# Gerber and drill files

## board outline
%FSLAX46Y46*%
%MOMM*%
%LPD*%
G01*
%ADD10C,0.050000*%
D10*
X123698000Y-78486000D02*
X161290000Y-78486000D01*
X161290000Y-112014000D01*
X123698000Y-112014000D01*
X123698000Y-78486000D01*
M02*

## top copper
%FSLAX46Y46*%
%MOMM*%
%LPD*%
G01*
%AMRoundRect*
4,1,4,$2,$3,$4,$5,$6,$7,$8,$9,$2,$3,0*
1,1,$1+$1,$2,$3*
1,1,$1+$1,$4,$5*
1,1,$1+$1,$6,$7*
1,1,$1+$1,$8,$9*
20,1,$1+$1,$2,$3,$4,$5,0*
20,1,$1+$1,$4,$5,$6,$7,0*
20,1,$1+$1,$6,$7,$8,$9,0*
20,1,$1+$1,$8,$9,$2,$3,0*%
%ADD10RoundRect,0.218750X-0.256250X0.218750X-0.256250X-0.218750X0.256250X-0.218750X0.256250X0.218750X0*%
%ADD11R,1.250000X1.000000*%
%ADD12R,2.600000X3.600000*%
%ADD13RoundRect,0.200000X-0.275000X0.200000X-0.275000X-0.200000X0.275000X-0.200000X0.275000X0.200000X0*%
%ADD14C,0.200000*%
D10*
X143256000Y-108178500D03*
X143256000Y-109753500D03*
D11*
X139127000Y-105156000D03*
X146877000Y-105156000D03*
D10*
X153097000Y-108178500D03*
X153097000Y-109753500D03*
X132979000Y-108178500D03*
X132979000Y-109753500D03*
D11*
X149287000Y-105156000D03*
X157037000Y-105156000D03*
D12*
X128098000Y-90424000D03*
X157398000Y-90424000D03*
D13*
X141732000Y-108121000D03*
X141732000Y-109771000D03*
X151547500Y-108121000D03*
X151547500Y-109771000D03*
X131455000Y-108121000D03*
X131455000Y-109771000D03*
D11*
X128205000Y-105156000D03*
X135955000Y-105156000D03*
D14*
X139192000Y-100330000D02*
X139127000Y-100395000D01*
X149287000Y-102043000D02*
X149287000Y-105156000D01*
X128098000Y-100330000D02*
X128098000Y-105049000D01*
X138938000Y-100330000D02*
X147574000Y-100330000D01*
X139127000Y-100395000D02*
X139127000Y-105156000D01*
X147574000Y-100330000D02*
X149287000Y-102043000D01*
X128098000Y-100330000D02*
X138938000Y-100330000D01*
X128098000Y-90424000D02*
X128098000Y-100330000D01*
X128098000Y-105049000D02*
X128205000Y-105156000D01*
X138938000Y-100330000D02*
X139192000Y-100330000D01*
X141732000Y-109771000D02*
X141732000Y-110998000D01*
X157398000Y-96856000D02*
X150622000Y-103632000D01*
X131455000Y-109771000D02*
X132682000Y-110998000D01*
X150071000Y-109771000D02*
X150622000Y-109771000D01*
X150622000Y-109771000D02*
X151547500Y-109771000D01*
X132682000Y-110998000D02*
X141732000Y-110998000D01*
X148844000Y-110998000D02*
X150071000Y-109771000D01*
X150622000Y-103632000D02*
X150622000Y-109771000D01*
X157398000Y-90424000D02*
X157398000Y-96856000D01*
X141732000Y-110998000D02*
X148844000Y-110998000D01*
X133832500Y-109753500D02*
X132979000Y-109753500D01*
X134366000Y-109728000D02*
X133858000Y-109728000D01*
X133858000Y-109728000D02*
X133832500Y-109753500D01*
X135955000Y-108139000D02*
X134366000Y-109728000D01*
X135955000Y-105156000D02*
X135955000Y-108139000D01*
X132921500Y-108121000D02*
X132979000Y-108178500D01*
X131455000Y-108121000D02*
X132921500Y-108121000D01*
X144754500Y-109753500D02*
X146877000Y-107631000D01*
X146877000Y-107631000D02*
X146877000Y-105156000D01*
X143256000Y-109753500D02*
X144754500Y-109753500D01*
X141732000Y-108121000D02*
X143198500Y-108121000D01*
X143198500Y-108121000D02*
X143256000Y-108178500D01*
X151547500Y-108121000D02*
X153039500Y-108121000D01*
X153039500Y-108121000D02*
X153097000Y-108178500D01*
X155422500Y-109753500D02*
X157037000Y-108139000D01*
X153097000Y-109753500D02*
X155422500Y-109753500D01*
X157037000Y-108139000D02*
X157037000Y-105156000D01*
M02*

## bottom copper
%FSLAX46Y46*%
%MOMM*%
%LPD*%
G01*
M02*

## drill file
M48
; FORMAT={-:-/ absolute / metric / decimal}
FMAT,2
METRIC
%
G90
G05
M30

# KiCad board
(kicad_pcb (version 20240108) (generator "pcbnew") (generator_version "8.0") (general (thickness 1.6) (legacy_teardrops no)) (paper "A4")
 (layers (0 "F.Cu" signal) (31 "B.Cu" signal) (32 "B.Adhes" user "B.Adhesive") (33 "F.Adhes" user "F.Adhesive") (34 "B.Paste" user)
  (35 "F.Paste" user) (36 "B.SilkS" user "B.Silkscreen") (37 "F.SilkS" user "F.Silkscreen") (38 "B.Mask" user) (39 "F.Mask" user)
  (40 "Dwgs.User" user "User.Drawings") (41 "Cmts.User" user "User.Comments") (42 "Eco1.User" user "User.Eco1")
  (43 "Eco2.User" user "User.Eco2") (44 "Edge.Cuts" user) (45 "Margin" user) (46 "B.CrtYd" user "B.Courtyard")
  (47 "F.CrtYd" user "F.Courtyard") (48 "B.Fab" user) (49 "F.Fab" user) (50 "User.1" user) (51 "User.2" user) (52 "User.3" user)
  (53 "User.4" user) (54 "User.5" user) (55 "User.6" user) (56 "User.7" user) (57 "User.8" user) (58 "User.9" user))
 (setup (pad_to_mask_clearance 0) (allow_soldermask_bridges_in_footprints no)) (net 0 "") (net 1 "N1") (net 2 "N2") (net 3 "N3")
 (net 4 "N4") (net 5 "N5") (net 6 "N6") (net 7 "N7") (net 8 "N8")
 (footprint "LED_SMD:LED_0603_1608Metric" (layer "F.Cu") (at 143.256 108.966 -90)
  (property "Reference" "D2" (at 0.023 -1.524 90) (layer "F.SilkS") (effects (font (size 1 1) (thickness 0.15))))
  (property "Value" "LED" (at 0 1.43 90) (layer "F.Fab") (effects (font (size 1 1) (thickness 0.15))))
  (pad "1" smd roundrect (at -0.7875 0 270) (size 0.875 0.95) (layers "F.Cu" "F.Paste" "F.Mask") (roundrect_rratio 0.25) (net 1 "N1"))
  (pad "2" smd roundrect (at 0.7875 0 270) (size 0.875 0.95) (layers "F.Cu" "F.Paste" "F.Mask") (roundrect_rratio 0.25) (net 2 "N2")))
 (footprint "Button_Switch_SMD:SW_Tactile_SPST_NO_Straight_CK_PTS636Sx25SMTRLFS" (layer "F.Cu") (at 143.002 105.156)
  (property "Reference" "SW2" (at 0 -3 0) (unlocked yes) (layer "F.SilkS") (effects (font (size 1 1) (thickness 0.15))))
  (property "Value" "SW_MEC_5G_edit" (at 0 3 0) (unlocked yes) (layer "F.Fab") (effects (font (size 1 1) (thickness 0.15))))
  (pad "1" smd rect (at -3.875 0) (size 1.25 1) (layers "F.Cu" "F.Paste" "F.Mask") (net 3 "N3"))
  (pad "2" smd rect (at 3.875 0) (size 1.25 1) (layers "F.Cu" "F.Paste" "F.Mask") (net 2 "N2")))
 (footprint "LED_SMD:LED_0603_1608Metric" (layer "F.Cu") (at 153.097 108.966 -90)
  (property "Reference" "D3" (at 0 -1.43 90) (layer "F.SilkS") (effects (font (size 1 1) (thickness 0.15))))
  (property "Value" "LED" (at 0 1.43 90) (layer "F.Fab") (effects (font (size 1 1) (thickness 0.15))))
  (pad "1" smd roundrect (at -0.7875 0 270) (size 0.875 0.95) (layers "F.Cu" "F.Paste" "F.Mask") (roundrect_rratio 0.25) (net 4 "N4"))
  (pad "2" smd roundrect (at 0.7875 0 270) (size 0.875 0.95) (layers "F.Cu" "F.Paste" "F.Mask") (roundrect_rratio 0.25) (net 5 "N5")))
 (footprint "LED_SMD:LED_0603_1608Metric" (layer "F.Cu") (at 132.979 108.966 -90)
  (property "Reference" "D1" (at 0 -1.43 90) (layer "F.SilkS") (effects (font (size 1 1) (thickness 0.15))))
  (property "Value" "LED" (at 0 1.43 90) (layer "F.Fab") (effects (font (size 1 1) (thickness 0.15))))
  (pad "1" smd roundrect (at -0.7875 0 270) (size 0.875 0.95) (layers "F.Cu" "F.Paste" "F.Mask") (roundrect_rratio 0.25) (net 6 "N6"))
  (pad "2" smd roundrect (at 0.7875 0 270) (size 0.875 0.95) (layers "F.Cu" "F.Paste" "F.Mask") (roundrect_rratio 0.25) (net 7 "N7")))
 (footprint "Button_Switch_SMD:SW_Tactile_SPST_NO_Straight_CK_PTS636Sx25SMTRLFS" (layer "F.Cu") (at 153.162 105.156)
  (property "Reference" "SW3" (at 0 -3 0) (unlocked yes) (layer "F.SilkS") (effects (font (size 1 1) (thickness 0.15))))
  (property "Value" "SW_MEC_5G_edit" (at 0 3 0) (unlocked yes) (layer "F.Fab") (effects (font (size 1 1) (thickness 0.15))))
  (pad "1" smd rect (at -3.875 0) (size 1.25 1) (layers "F.Cu" "F.Paste" "F.Mask") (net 3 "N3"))
  (pad "2" smd rect (at 3.875 0) (size 1.25 1) (layers "F.Cu" "F.Paste" "F.Mask") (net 5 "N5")))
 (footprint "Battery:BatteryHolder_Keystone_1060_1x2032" (layer "F.Cu") (at 142.748 90.424)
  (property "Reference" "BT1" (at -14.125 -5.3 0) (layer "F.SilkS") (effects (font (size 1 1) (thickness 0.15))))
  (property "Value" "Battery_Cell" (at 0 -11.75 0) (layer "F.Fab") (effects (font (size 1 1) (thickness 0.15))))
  (pad "1" smd rect (at -14.65 0 180) (size 2.6 3.6) (layers "F.Cu" "F.Paste" "F.Mask") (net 3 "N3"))
  (pad "2" smd rect (at 14.65 0 180) (size 2.6 3.6) (layers "F.Cu" "F.Paste" "F.Mask") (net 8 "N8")))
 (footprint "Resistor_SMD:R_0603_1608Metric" (layer "F.Cu") (at 141.732 108.946 -90)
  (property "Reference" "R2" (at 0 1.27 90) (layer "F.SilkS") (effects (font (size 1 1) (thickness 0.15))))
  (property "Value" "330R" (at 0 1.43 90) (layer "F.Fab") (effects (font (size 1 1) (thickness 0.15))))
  (pad "1" smd roundrect (at -0.825 0 270) (size 0.8 0.95) (layers "F.Cu" "F.Paste" "F.Mask") (roundrect_rratio 0.25) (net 1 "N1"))
  (pad "2" smd roundrect (at 0.825 0 270) (size 0.8 0.95) (layers "F.Cu" "F.Paste" "F.Mask") (roundrect_rratio 0.25) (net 8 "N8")))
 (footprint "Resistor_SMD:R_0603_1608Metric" (layer "F.Cu") (at 151.5475 108.946 -90)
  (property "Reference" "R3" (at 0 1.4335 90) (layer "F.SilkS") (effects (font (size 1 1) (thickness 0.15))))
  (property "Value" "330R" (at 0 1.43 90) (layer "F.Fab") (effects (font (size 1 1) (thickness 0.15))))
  (pad "1" smd roundrect (at -0.825 0 270) (size 0.8 0.95) (layers "F.Cu" "F.Paste" "F.Mask") (roundrect_rratio 0.25) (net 4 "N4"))
  (pad "2" smd roundrect (at 0.825 0 270) (size 0.8 0.95) (layers "F.Cu" "F.Paste" "F.Mask") (roundrect_rratio 0.25) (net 8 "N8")))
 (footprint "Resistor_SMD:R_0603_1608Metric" (layer "F.Cu") (at 131.455 108.946 -90)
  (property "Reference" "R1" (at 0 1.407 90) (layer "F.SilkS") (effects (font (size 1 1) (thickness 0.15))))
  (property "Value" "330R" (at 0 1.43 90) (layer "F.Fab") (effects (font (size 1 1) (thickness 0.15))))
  (pad "1" smd roundrect (at -0.825 0 270) (size 0.8 0.95) (layers "F.Cu" "F.Paste" "F.Mask") (roundrect_rratio 0.25) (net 6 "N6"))
  (pad "2" smd roundrect (at 0.825 0 270) (size 0.8 0.95) (layers "F.Cu" "F.Paste" "F.Mask") (roundrect_rratio 0.25) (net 8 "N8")))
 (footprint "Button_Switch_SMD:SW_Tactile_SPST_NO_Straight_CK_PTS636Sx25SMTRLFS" (layer "F.Cu") (at 132.08 105.156)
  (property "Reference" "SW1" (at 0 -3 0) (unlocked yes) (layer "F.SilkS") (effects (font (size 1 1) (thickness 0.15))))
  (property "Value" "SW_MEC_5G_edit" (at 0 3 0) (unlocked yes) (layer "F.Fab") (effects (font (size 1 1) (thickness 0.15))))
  (pad "1" smd rect (at -3.875 0) (size 1.25 1) (layers "F.Cu" "F.Paste" "F.Mask") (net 3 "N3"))
  (pad "2" smd rect (at 3.875 0) (size 1.25 1) (layers "F.Cu" "F.Paste" "F.Mask") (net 7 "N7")))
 (gr_rect (start 123.698 78.486) (end 161.29 112.014) (stroke (width 0.05) (type default)) (fill none) (layer "Edge.Cuts"))
 (segment (start 139.192 100.33) (end 139.127 100.395) (width 0.2) (layer "F.Cu") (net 3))
 (segment (start 149.287 102.043) (end 149.287 105.156) (width 0.2) (layer "F.Cu") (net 3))
 (segment (start 128.098 100.33) (end 128.098 105.049) (width 0.2) (layer "F.Cu") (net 3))
 (segment (start 138.938 100.33) (end 147.574 100.33) (width 0.2) (layer "F.Cu") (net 3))
 (segment (start 139.127 100.395) (end 139.127 105.156) (width 0.2) (layer "F.Cu") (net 3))
 (segment (start 147.574 100.33) (end 149.287 102.043) (width 0.2) (layer "F.Cu") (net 3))
 (segment (start 128.098 100.33) (end 138.938 100.33) (width 0.2) (layer "F.Cu") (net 3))
 (segment (start 128.098 90.424) (end 128.098 100.33) (width 0.2) (layer "F.Cu") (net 3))
 (segment (start 128.098 105.049) (end 128.205 105.156) (width 0.2) (layer "F.Cu") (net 3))
 (segment (start 138.938 100.33) (end 139.192 100.33) (width 0.2) (layer "F.Cu") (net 3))
 (segment (start 141.732 109.771) (end 141.732 110.998) (width 0.2) (layer "F.Cu") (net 8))
 (segment (start 157.398 96.856) (end 150.622 103.632) (width 0.2) (layer "F.Cu") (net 8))
 (segment (start 131.455 109.771) (end 132.682 110.998) (width 0.2) (layer "F.Cu") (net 8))
 (segment (start 150.071 109.771) (end 150.622 109.771) (width 0.2) (layer "F.Cu") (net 8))
 (segment (start 150.622 109.771) (end 151.5475 109.771) (width 0.2) (layer "F.Cu") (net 8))
 (segment (start 132.682 110.998) (end 141.732 110.998) (width 0.2) (layer "F.Cu") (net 8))
 (segment (start 148.844 110.998) (end 150.071 109.771) (width 0.2) (layer "F.Cu") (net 8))
 (segment (start 150.622 103.632) (end 150.622 109.771) (width 0.2) (layer "F.Cu") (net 8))
 (segment (start 157.398 90.424) (end 157.398 96.856) (width 0.2) (layer "F.Cu") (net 8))
 (segment (start 141.732 110.998) (end 148.844 110.998) (width 0.2) (layer "F.Cu") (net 8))
 (segment (start 133.8325 109.7535) (end 132.979 109.7535) (width 0.2) (layer "F.Cu") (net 7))
 (segment (start 134.366 109.728) (end 133.858 109.728) (width 0.2) (layer "F.Cu") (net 7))
 (segment (start 133.858 109.728) (end 133.8325 109.7535) (width 0.2) (layer "F.Cu") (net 7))
 (segment (start 135.955 108.139) (end 134.366 109.728) (width 0.2) (layer "F.Cu") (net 7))
 (segment (start 135.955 105.156) (end 135.955 108.139) (width 0.2) (layer "F.Cu") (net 7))
 (segment (start 132.9215 108.121) (end 132.979 108.1785) (width 0.2) (layer "F.Cu") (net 6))
 (segment (start 131.455 108.121) (end 132.9215 108.121) (width 0.2) (layer "F.Cu") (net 6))
 (segment (start 144.7545 109.7535) (end 146.877 107.631) (width 0.2) (layer "F.Cu") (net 2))
 (segment (start 146.877 107.631) (end 146.877 105.156) (width 0.2) (layer "F.Cu") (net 2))
 (segment (start 143.256 109.7535) (end 144.7545 109.7535) (width 0.2) (layer "F.Cu") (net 2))
 (segment (start 141.732 108.121) (end 143.1985 108.121) (width 0.2) (layer "F.Cu") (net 1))
 (segment (start 143.1985 108.121) (end 143.256 108.1785) (width 0.2) (layer "F.Cu") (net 1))
 (segment (start 151.5475 108.121) (end 153.0395 108.121) (width 0.2) (layer "F.Cu") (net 4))
 (segment (start 153.0395 108.121) (end 153.097 108.1785) (width 0.2) (layer "F.Cu") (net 4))
 (segment (start 155.4225 109.7535) (end 157.037 108.139) (width 0.2) (layer "F.Cu") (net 5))
 (segment (start 153.097 109.7535) (end 155.4225 109.7535) (width 0.2) (layer "F.Cu") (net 5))
 (segment (start 157.037 108.139) (end 157.037 105.156) (width 0.2) (layer "F.Cu") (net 5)))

